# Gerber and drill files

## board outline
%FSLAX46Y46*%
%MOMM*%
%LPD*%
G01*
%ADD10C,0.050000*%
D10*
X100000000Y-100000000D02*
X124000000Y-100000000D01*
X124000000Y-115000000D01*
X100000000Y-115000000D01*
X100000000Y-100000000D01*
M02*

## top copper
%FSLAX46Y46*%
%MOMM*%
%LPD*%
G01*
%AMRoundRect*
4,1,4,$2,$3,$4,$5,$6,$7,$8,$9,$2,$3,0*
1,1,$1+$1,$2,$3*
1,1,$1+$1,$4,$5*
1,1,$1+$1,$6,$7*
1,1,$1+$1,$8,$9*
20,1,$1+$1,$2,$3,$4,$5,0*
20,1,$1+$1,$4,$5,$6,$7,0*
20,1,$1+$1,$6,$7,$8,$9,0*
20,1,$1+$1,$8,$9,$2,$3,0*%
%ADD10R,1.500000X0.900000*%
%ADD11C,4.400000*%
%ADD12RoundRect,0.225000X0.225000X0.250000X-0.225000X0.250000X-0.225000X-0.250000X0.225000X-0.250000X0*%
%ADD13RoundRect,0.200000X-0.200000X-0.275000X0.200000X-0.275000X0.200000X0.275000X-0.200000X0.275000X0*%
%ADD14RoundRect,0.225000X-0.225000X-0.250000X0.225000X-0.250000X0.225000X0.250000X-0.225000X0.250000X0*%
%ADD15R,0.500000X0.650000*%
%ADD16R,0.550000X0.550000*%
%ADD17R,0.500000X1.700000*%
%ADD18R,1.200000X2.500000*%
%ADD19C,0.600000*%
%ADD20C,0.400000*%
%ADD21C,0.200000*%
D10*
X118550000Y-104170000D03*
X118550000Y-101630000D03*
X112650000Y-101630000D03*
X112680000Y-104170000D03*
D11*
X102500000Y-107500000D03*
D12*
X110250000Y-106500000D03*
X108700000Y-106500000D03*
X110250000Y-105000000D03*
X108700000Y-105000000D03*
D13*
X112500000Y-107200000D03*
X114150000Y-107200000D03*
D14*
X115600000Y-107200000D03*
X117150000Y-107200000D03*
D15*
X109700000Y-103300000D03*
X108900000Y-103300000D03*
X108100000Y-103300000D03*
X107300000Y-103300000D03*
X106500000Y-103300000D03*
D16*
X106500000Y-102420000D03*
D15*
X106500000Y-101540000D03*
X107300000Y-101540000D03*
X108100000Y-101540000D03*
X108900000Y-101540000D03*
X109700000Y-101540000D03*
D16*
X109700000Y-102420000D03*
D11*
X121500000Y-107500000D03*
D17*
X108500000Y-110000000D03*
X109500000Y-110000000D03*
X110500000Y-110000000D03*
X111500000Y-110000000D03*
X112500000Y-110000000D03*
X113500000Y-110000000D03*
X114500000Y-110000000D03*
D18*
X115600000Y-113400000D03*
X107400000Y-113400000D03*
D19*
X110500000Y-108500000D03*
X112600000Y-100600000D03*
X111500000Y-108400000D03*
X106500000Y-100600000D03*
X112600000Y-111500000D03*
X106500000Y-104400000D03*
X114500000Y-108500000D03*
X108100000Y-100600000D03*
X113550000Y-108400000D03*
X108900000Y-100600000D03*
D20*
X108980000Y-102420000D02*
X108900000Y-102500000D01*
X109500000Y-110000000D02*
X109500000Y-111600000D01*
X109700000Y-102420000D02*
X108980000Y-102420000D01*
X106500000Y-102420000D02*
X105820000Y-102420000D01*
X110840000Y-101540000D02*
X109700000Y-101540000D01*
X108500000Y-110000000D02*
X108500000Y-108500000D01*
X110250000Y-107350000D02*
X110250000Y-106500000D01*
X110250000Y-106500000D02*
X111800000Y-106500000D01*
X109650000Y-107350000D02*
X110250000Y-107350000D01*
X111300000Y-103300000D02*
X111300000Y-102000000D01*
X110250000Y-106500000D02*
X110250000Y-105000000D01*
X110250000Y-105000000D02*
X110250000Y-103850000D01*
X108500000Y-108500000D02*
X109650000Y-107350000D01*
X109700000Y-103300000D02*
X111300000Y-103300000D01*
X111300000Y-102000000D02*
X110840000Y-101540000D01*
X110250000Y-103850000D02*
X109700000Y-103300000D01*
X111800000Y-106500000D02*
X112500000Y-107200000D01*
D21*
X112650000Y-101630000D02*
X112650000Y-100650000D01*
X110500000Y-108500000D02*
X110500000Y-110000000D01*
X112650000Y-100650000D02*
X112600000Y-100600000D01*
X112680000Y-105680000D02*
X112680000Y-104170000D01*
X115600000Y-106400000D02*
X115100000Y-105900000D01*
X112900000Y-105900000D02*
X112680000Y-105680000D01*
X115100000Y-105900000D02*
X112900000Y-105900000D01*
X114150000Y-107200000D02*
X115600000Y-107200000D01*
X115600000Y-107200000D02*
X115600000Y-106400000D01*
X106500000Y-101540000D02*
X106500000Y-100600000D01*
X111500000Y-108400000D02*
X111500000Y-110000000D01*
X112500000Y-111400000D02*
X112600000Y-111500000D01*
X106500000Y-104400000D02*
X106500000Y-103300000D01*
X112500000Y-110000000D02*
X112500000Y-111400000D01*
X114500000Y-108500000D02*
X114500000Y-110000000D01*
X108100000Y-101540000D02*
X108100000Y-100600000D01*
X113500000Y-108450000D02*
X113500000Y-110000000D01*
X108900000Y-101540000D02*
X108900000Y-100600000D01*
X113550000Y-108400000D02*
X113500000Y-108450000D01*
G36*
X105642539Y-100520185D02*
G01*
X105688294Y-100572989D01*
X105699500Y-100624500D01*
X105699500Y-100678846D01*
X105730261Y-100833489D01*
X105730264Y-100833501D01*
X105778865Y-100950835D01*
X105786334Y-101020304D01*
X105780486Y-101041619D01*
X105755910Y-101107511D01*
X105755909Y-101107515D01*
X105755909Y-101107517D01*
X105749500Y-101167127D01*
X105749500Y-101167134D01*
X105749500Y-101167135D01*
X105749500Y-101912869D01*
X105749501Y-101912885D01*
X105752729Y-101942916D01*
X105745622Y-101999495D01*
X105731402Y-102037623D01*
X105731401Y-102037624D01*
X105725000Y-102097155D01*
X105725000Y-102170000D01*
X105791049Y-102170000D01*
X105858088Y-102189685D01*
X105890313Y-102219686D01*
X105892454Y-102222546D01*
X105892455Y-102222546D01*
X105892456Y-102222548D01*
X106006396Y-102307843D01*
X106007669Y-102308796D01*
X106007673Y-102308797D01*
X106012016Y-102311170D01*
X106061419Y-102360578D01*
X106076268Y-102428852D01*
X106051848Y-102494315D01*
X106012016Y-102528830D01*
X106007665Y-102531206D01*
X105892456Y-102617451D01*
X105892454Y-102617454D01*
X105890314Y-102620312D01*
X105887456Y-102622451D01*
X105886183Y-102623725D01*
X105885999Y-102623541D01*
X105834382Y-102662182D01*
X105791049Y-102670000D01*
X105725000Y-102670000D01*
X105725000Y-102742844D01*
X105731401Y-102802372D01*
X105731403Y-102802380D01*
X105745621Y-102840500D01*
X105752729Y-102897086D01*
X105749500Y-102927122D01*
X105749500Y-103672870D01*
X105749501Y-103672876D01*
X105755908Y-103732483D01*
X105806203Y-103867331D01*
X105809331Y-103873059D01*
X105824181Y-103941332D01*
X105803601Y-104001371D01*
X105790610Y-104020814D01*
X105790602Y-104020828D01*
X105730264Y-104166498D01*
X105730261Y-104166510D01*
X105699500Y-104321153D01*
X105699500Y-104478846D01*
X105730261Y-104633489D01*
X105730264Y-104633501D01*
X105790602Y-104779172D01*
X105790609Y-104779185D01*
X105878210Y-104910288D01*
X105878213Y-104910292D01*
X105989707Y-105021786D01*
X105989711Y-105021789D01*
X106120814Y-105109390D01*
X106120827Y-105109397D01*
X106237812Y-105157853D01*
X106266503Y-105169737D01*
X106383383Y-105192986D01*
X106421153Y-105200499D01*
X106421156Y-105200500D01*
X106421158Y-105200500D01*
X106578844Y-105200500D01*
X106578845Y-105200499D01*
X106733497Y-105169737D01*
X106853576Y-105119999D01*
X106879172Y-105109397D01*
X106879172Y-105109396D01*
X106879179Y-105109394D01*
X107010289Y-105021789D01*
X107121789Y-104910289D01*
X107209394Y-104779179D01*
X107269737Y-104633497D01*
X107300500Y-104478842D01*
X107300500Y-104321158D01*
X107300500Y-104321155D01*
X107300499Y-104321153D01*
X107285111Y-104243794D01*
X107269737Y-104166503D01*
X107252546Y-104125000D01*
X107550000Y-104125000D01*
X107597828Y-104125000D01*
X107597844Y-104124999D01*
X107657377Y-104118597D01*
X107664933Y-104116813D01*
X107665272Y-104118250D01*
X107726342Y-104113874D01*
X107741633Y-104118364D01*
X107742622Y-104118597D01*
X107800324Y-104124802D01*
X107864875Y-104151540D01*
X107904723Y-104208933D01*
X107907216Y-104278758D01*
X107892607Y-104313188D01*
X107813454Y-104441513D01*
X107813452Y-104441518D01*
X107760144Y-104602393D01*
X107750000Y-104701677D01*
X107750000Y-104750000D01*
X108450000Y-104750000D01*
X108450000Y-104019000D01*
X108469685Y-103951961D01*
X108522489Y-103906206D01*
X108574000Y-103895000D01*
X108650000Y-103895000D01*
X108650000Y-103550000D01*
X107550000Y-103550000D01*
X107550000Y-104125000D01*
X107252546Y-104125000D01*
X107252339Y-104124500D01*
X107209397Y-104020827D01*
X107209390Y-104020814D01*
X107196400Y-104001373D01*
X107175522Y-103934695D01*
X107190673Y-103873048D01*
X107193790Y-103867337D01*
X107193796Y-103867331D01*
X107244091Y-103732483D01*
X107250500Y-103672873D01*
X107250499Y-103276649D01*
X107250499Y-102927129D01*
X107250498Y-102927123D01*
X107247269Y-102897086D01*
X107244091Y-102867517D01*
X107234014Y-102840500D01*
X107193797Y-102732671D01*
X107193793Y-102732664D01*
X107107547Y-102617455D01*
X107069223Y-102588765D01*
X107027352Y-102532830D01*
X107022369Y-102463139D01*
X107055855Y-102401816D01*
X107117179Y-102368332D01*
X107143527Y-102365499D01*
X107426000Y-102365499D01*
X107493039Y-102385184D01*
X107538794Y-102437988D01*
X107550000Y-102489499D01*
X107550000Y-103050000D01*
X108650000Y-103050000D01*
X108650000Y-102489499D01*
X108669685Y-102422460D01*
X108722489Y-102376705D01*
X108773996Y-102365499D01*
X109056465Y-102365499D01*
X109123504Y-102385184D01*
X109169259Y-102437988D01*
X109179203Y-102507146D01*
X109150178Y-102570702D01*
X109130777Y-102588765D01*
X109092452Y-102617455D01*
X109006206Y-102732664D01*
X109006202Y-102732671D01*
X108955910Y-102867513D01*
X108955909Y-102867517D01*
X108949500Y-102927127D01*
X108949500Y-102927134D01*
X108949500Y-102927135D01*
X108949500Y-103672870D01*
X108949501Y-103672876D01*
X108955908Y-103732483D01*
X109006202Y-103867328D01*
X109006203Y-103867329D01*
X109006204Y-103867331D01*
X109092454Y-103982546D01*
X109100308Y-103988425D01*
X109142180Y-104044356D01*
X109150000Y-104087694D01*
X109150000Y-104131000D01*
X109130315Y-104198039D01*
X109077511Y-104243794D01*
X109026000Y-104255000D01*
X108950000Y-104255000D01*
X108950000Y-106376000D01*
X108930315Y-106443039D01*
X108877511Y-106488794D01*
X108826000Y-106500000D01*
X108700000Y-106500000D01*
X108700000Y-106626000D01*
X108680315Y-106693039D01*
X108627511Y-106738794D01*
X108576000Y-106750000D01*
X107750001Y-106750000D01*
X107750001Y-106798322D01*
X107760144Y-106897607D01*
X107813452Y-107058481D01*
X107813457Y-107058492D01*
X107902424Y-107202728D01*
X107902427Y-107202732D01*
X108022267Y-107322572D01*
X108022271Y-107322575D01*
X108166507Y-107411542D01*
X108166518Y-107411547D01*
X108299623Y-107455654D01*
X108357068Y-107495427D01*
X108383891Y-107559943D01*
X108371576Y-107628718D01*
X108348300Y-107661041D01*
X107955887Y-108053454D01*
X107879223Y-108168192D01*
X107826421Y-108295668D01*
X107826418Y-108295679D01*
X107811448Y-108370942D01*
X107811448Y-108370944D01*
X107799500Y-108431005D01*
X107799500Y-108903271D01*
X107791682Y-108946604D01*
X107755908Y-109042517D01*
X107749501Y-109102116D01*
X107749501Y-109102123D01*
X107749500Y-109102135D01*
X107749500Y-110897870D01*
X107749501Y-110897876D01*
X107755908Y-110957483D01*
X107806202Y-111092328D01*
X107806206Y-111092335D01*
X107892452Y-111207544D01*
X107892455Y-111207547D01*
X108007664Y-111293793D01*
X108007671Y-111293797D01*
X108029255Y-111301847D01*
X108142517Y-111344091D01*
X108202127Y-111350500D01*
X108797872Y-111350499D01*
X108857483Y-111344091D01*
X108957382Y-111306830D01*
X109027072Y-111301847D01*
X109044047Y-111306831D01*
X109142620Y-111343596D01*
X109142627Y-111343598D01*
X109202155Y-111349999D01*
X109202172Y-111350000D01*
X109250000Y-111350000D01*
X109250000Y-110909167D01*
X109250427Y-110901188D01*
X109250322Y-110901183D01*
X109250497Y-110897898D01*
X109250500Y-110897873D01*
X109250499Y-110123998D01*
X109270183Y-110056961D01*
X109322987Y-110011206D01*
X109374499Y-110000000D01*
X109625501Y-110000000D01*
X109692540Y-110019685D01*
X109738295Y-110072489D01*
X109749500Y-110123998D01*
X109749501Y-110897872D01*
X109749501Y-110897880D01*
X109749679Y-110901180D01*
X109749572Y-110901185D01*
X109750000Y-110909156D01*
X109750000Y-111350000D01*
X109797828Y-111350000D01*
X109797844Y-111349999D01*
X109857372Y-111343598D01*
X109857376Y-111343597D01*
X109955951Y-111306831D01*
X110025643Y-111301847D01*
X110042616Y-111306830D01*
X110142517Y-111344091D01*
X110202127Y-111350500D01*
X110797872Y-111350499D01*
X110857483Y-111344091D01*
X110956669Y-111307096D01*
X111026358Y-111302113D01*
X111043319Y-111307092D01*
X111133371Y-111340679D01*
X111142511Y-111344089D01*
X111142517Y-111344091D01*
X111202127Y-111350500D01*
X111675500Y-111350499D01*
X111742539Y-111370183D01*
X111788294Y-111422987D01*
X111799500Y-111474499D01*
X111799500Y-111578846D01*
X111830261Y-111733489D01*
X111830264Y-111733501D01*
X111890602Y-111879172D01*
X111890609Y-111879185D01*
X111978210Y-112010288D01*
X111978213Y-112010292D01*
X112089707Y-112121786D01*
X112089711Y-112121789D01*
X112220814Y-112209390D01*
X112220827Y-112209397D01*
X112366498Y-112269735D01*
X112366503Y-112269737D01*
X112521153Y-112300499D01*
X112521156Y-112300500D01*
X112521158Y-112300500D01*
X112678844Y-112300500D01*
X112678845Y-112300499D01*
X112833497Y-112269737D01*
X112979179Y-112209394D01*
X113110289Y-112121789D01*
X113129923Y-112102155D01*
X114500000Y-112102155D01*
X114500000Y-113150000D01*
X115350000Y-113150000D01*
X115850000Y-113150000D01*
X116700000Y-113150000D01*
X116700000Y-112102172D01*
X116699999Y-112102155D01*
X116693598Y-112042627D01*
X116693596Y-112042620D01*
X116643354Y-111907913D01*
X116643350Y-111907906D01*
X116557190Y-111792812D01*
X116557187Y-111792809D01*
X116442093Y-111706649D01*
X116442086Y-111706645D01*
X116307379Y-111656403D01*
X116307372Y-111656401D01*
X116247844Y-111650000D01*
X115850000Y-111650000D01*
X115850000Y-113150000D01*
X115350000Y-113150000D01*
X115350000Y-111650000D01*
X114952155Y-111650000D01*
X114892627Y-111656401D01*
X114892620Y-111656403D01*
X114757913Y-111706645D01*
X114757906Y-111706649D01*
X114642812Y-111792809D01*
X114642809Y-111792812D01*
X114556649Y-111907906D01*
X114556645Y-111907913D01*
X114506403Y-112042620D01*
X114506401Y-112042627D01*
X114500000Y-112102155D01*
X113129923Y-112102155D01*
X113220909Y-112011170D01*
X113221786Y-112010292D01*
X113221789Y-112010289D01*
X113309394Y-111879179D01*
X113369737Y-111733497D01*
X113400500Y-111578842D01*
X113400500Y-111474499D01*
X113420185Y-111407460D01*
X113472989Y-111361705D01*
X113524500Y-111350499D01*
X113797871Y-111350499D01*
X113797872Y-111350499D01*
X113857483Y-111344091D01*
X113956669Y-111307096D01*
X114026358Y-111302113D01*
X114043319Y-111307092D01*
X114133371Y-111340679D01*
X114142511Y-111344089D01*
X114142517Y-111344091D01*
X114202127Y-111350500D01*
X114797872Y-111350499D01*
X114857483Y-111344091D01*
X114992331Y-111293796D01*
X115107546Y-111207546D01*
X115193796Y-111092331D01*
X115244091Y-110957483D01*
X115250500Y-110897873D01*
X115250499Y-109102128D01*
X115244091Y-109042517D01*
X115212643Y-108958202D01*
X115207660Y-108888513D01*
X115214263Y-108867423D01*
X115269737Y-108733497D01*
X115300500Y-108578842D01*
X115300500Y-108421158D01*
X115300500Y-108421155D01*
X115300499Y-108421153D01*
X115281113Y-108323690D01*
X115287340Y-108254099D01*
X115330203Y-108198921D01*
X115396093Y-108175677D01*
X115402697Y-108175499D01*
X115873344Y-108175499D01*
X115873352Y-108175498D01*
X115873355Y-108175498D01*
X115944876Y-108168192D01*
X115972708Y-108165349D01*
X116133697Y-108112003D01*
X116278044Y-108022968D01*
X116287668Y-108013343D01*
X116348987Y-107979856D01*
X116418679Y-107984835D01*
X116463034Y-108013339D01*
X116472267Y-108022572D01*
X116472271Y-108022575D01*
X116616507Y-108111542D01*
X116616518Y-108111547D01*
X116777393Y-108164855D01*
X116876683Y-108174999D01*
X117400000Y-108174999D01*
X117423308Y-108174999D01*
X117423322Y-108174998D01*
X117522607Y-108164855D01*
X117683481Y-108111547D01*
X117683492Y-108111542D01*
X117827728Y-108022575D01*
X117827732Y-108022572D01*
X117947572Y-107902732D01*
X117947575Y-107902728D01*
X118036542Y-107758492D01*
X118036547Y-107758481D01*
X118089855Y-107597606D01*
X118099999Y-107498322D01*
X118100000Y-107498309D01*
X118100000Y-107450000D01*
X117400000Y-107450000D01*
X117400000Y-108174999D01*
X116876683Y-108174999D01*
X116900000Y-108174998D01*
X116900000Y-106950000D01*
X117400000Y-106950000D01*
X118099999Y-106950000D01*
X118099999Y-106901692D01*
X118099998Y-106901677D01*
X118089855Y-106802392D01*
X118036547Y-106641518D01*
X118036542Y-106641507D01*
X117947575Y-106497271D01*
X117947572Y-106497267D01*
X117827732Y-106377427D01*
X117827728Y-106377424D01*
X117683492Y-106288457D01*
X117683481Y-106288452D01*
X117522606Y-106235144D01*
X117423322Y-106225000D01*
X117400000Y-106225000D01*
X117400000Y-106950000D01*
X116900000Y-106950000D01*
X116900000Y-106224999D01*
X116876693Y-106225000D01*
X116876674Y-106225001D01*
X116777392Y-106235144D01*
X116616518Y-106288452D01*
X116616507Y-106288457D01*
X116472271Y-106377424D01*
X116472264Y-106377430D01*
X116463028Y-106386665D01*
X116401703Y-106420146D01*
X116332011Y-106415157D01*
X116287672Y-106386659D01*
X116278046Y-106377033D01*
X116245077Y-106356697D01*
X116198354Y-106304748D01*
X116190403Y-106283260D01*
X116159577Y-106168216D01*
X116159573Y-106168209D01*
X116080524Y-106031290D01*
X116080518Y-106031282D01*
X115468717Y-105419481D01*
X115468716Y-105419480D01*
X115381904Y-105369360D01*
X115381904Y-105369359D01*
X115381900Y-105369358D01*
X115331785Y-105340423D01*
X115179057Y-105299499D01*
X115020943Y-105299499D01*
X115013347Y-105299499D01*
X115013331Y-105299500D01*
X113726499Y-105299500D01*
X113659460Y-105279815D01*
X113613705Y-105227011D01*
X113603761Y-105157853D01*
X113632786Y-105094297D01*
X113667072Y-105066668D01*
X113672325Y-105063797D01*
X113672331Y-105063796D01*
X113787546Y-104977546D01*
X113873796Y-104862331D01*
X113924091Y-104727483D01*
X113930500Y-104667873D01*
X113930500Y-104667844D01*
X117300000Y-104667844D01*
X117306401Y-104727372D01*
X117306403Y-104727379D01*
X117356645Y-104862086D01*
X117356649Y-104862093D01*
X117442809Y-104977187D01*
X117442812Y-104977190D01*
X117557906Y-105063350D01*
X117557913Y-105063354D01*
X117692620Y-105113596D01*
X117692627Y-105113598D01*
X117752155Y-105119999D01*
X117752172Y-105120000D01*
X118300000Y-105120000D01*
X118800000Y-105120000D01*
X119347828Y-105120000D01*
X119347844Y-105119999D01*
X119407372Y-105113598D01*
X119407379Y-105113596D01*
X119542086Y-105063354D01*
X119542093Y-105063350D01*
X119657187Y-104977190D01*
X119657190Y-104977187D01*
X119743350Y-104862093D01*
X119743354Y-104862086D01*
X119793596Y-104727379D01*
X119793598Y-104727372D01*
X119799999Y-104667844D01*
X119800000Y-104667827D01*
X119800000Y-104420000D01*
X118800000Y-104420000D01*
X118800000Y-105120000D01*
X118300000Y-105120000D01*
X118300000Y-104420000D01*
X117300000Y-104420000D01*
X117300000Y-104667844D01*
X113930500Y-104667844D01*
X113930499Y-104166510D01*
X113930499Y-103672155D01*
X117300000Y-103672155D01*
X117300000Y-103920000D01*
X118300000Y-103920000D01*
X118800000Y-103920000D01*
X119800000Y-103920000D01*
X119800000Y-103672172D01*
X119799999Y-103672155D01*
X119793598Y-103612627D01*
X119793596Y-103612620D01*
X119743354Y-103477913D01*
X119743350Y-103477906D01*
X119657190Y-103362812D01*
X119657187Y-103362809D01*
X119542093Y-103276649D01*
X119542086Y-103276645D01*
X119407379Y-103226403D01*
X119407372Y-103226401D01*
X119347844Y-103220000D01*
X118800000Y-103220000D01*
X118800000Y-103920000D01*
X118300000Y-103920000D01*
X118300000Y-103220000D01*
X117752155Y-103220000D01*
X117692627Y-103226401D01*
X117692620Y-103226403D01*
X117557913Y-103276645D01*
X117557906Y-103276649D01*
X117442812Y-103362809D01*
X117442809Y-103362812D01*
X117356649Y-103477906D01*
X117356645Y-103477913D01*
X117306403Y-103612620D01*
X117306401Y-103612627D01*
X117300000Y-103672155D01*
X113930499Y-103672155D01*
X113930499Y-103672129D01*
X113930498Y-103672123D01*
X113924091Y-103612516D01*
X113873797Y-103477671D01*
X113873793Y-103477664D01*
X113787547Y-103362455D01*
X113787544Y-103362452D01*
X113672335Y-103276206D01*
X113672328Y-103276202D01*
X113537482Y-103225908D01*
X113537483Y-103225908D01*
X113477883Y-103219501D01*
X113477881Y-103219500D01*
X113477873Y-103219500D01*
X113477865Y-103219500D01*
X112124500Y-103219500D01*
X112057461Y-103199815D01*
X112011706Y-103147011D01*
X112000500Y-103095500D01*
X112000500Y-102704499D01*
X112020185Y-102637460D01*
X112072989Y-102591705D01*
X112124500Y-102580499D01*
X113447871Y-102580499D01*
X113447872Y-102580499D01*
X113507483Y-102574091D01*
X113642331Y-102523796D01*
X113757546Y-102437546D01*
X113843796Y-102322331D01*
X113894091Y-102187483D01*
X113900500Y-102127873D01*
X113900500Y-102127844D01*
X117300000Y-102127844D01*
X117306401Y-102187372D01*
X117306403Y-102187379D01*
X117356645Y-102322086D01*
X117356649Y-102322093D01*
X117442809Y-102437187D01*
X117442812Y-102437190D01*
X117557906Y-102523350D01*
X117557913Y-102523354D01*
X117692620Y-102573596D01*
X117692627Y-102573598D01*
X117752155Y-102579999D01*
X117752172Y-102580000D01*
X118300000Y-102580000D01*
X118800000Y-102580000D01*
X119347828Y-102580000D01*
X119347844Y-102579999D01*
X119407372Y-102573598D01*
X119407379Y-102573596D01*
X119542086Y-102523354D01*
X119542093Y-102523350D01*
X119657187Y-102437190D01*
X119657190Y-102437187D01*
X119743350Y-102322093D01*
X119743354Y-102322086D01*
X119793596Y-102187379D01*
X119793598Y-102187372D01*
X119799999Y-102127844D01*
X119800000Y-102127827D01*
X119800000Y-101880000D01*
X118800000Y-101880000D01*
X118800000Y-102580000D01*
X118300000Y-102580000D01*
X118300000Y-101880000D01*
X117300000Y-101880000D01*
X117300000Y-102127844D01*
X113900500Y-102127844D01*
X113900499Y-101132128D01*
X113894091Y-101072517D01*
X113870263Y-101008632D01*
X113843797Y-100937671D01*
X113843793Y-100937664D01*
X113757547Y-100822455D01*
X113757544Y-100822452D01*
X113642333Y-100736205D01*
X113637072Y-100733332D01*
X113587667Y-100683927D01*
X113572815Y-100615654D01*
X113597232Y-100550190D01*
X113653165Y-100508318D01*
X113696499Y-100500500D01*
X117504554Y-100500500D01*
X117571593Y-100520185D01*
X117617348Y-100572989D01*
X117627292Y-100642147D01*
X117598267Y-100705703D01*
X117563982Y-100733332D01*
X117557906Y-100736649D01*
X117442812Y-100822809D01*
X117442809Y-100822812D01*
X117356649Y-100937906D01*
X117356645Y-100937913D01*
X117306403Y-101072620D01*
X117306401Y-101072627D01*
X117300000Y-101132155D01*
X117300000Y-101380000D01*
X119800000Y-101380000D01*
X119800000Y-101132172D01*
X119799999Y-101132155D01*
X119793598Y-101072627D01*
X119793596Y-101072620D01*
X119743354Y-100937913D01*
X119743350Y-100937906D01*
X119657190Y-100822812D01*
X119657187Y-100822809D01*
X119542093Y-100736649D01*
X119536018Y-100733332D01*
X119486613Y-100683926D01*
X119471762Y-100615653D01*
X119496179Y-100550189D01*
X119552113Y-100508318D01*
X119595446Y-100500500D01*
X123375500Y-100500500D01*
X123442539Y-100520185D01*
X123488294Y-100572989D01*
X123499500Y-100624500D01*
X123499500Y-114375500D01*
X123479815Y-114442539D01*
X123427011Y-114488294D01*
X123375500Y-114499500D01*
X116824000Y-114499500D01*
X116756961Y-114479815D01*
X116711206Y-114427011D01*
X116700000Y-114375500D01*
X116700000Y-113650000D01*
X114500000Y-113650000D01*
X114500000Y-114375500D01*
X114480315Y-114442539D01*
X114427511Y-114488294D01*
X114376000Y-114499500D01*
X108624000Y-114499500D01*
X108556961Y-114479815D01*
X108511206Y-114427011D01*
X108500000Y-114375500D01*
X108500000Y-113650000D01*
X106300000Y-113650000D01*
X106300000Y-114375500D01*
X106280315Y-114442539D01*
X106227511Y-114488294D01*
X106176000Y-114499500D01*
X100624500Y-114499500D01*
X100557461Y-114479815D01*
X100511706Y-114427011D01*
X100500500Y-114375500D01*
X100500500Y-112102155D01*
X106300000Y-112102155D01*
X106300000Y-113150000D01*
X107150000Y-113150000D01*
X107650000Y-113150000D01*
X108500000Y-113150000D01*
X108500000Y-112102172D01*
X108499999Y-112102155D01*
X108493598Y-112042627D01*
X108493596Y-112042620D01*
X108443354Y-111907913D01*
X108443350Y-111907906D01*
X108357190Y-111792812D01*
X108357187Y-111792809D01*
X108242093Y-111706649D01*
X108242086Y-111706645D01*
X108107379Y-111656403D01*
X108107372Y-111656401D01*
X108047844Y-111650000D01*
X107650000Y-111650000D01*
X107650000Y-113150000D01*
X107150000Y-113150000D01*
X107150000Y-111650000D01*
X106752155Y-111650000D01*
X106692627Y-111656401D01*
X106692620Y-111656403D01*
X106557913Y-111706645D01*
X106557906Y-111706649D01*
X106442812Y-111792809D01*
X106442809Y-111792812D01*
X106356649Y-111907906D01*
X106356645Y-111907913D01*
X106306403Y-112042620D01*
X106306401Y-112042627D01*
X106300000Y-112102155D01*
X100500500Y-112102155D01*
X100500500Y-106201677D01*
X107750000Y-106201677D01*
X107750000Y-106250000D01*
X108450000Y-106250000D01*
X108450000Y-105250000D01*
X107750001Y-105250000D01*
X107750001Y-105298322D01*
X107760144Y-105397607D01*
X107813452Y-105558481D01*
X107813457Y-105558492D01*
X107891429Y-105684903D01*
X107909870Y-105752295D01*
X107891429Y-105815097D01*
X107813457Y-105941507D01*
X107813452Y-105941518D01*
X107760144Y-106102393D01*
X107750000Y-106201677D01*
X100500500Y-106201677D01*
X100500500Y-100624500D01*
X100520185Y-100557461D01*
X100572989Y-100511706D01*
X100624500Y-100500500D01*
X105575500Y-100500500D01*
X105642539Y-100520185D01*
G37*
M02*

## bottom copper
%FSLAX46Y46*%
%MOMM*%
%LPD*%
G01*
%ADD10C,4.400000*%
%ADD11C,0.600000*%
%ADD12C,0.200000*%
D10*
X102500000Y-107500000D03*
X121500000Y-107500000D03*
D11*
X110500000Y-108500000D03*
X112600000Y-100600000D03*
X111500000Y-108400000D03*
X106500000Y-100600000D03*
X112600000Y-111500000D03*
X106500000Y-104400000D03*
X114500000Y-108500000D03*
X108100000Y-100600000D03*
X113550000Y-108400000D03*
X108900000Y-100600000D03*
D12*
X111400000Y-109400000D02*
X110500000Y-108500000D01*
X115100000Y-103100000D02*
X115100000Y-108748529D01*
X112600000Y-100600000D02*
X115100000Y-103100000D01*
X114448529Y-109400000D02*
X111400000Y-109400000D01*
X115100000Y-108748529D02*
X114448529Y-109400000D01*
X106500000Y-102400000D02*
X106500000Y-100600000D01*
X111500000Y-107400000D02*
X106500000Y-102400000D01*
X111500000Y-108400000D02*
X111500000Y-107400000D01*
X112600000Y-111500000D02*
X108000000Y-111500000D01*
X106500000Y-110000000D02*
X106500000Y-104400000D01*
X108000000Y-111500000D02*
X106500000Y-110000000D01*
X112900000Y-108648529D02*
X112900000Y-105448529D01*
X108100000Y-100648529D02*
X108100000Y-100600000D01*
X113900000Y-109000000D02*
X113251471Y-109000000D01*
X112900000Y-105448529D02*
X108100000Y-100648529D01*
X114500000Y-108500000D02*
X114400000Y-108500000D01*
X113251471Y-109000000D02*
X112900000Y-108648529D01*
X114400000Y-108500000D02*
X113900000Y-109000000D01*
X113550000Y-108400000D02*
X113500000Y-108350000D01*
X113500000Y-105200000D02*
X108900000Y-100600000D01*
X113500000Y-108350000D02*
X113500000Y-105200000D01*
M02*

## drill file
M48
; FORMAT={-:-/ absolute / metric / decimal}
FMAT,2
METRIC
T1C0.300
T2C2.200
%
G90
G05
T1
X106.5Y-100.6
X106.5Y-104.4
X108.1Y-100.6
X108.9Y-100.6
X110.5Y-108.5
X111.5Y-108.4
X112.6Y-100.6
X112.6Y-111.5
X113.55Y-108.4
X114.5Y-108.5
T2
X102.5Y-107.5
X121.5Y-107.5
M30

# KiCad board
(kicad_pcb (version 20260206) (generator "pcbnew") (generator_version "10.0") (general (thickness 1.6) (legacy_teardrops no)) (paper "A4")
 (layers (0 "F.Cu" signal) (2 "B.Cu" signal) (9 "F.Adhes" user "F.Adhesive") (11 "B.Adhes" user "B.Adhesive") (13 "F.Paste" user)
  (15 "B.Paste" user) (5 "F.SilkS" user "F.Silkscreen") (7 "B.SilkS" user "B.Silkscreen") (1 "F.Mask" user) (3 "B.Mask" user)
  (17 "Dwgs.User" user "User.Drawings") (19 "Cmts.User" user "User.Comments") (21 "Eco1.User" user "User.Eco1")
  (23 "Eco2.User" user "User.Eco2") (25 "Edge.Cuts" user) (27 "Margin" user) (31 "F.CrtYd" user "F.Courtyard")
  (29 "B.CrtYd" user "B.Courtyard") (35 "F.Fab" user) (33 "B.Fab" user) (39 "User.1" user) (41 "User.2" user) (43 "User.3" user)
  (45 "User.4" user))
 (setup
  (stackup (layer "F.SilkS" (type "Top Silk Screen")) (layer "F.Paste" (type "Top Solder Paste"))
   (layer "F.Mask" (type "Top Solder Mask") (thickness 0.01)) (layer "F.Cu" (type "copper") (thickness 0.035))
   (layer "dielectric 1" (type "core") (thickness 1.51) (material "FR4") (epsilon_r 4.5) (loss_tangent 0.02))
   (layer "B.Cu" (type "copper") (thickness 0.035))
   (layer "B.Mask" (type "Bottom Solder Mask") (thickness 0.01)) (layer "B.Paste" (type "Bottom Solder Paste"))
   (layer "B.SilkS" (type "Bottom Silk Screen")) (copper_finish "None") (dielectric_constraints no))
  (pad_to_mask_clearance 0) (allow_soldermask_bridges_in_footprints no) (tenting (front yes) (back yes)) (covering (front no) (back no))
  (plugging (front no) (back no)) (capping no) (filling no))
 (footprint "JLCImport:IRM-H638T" (layer "F.Cu") (at 115.6 102.9 180)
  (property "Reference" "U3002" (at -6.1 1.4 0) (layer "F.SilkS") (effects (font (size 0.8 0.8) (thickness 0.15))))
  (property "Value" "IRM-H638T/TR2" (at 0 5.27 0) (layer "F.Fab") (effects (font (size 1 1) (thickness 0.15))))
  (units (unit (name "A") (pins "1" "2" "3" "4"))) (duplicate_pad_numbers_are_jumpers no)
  (pad "1" smd rect (at -2.95 -1.27 270) (size 0.9 1.5) (layers "F.Cu" "F.Mask" "F.Paste") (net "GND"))
  (pad "2" smd rect (at -2.95 1.27 270) (size 0.9 1.5) (layers "F.Cu" "F.Mask" "F.Paste") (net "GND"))
  (pad "3" smd rect (at 2.95 1.27 270) (size 0.9 1.5) (layers "F.Cu" "F.Mask" "F.Paste") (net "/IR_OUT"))
  (pad "4" smd rect (at 2.92 -1.27 270) (size 0.9 1.5) (layers "F.Cu" "F.Mask" "F.Paste") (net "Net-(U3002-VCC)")))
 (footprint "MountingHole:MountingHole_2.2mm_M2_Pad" (layer "F.Cu") (at 102.5 107.5)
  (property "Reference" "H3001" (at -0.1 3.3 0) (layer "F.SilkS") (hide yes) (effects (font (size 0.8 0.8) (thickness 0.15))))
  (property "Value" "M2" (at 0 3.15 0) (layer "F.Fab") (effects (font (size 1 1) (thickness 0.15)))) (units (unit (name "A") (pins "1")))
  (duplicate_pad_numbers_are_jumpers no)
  (pad "1" thru_hole circle (at 0 0) (size 4.4 4.4) (drill 2.2) (layers "*.Cu" "*.Mask") (remove_unused_layers no) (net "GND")
   (zone_connect 2)))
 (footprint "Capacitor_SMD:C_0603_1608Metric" (layer "F.Cu") (at 109.475 106.5 180)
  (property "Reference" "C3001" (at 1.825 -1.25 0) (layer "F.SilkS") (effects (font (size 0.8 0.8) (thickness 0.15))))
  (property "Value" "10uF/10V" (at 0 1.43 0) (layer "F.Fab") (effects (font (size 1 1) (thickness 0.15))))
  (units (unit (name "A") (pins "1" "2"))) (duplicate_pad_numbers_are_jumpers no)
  (pad "1" smd roundrect (at -0.775 0 180) (size 0.9 0.95) (layers "F.Cu" "F.Mask" "F.Paste") (roundrect_rratio 0.25) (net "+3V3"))
  (pad "2" smd roundrect (at 0.775 0 180) (size 0.9 0.95) (layers "F.Cu" "F.Mask" "F.Paste") (roundrect_rratio 0.25) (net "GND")))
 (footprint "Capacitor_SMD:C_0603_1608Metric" (layer "F.Cu") (at 109.475 105 180)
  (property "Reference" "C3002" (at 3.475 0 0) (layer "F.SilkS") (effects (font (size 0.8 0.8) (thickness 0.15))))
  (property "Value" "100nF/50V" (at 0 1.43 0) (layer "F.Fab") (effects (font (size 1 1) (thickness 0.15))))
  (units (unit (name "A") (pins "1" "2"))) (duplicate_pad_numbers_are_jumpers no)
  (pad "1" smd roundrect (at -0.775 0 180) (size 0.9 0.95) (layers "F.Cu" "F.Mask" "F.Paste") (roundrect_rratio 0.25) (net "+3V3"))
  (pad "2" smd roundrect (at 0.775 0 180) (size 0.9 0.95) (layers "F.Cu" "F.Mask" "F.Paste") (roundrect_rratio 0.25) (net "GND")))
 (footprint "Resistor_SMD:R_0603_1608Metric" (layer "F.Cu") (at 113.325 107.2)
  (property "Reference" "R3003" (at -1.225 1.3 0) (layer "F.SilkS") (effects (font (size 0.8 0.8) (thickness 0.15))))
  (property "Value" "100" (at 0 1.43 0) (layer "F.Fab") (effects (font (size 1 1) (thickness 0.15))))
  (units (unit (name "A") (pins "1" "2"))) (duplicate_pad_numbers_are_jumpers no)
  (pad "1" smd roundrect (at -0.825 0) (size 0.8 0.95) (layers "F.Cu" "F.Mask" "F.Paste") (roundrect_rratio 0.25) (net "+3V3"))
  (pad "2" smd roundrect (at 0.825 0) (size 0.8 0.95) (layers "F.Cu" "F.Mask" "F.Paste") (roundrect_rratio 0.25) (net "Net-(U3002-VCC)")))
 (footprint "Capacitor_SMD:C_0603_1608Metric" (layer "F.Cu") (at 116.375 107.2)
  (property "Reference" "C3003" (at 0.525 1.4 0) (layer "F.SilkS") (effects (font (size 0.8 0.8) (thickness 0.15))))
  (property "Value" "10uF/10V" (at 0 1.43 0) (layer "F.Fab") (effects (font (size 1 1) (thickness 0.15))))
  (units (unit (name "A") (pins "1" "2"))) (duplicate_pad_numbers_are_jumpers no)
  (pad "1" smd roundrect (at -0.775 0) (size 0.9 0.95) (layers "F.Cu" "F.Mask" "F.Paste") (roundrect_rratio 0.25) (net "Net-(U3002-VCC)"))
  (pad "2" smd roundrect (at 0.775 0) (size 0.9 0.95) (layers "F.Cu" "F.Mask" "F.Paste") (roundrect_rratio 0.25) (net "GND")))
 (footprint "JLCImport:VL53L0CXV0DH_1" (layer "F.Cu") (at 108.1 102.42)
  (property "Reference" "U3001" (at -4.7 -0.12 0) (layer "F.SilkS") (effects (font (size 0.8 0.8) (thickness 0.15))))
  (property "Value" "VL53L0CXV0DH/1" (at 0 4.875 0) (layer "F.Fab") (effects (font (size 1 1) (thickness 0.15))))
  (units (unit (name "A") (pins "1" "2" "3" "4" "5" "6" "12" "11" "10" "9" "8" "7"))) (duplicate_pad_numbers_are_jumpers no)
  (pad "1" smd rect (at 1.6 0.88) (size 0.5 0.65) (layers "F.Cu" "F.Mask" "F.Paste") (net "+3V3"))
  (pad "2" smd rect (at 0.8 0.88) (size 0.5 0.65) (layers "F.Cu" "F.Mask" "F.Paste") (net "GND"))
  (pad "3" smd rect (at 0 0.88) (size 0.5 0.65) (layers "F.Cu" "F.Mask" "F.Paste") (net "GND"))
  (pad "4" smd rect (at -0.8 0.88) (size 0.5 0.65) (layers "F.Cu" "F.Mask" "F.Paste") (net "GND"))
  (pad "5" smd rect (at -1.6 0.88) (size 0.5 0.65) (layers "F.Cu" "F.Mask" "F.Paste") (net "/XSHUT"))
  (pad "6" smd rect (at -1.6 0) (size 0.55 0.55) (layers "F.Cu" "F.Mask" "F.Paste") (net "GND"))
  (pad "7" smd rect (at -1.6 -0.88) (size 0.5 0.65) (layers "F.Cu" "F.Mask" "F.Paste") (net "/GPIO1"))
  (pad "8" smd rect (at -0.8 -0.88) (size 0.5 0.65) (layers "F.Cu" "F.Mask" "F.Paste") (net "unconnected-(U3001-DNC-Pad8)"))
  (pad "9" smd rect (at 0 -0.88) (size 0.5 0.65) (layers "F.Cu" "F.Mask" "F.Paste") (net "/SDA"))
  (pad "10" smd rect (at 0.8 -0.88) (size 0.5 0.65) (layers "F.Cu" "F.Mask" "F.Paste") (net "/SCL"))
  (pad "11" smd rect (at 1.6 -0.88) (size 0.5 0.65) (layers "F.Cu" "F.Mask" "F.Paste") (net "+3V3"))
  (pad "12" smd rect (at 1.6 0) (size 0.55 0.55) (layers "F.Cu" "F.Mask" "F.Paste") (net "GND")))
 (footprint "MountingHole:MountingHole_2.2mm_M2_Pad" (layer "F.Cu") (at 121.5 107.5)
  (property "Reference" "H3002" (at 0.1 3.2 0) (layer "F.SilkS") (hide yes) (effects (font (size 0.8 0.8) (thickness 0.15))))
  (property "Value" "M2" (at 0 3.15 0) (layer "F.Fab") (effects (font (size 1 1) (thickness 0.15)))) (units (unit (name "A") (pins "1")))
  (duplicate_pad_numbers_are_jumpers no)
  (pad "1" thru_hole circle (at 0 0) (size 4.4 4.4) (drill 2.2) (layers "*.Cu" "*.Mask") (remove_unused_layers no) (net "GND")
   (zone_connect 2)))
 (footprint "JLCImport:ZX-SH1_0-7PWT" (layer "F.Cu") (at 111.5 111.7)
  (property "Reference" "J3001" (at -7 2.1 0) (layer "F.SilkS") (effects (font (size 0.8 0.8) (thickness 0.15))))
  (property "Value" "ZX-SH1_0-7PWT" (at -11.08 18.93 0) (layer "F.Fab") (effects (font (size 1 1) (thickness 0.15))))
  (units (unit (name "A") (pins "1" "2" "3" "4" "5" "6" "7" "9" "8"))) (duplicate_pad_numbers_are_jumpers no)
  (pad "1" smd rect (at -3 -1.7) (size 0.5 1.7) (layers "F.Cu" "F.Mask" "F.Paste") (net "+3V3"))
  (pad "2" smd rect (at -2 -1.7) (size 0.5 1.7) (layers "F.Cu" "F.Mask" "F.Paste") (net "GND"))
  (pad "3" smd rect (at -1 -1.7) (size 0.5 1.7) (layers "F.Cu" "F.Mask" "F.Paste") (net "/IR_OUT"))
  (pad "4" smd rect (at 0 -1.7) (size 0.5 1.7) (layers "F.Cu" "F.Mask" "F.Paste") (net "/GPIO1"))
  (pad "5" smd rect (at 1 -1.7) (size 0.5 1.7) (layers "F.Cu" "F.Mask" "F.Paste") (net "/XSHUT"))
  (pad "6" smd rect (at 2 -1.7) (size 0.5 1.7) (layers "F.Cu" "F.Mask" "F.Paste") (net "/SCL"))
  (pad "7" smd rect (at 3 -1.7) (size 0.5 1.7) (layers "F.Cu" "F.Mask" "F.Paste") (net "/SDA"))
  (pad "8" smd rect (at 4.1 1.7) (size 1.2 2.5) (layers "F.Cu" "F.Mask" "F.Paste") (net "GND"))
  (pad "9" smd rect (at -4.1 1.7) (size 1.2 2.5) (layers "F.Cu" "F.Mask" "F.Paste") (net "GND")))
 (gr_rect (start 100 100) (end 124 115) (stroke (width 0.05) (type solid)) (fill no) (layer "Edge.Cuts"))
 (segment (start 108.98 102.42) (end 108.9 102.5) (width 0.4) (layer "F.Cu") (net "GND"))
 (segment (start 109.5 110) (end 109.5 111.6) (width 0.4) (layer "F.Cu") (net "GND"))
 (segment (start 109.7 102.42) (end 108.98 102.42) (width 0.4) (layer "F.Cu") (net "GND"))
 (segment (start 106.5 102.42) (end 105.82 102.42) (width 0.4) (layer "F.Cu") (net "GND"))
 (segment (start 110.84 101.54) (end 109.7 101.54) (width 0.4) (layer "F.Cu") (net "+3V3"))
 (segment (start 108.5 110) (end 108.5 108.5) (width 0.4) (layer "F.Cu") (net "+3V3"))
 (segment (start 110.25 107.35) (end 110.25 106.5) (width 0.4) (layer "F.Cu") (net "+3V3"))
 (segment (start 110.25 106.5) (end 111.8 106.5) (width 0.4) (layer "F.Cu") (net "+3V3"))
 (segment (start 109.65 107.35) (end 110.25 107.35) (width 0.4) (layer "F.Cu") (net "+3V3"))
 (segment (start 111.3 103.3) (end 111.3 102) (width 0.4) (layer "F.Cu") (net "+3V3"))
 (segment (start 110.25 106.5) (end 110.25 105) (width 0.4) (layer "F.Cu") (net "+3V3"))
 (segment (start 110.25 105) (end 110.25 103.85) (width 0.4) (layer "F.Cu") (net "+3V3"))
 (segment (start 108.5 108.5) (end 109.65 107.35) (width 0.4) (layer "F.Cu") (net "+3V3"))
 (segment (start 109.7 103.3) (end 111.3 103.3) (width 0.4) (layer "F.Cu") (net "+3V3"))
 (segment (start 111.3 102) (end 110.84 101.54) (width 0.4) (layer "F.Cu") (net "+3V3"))
 (segment (start 110.25 103.85) (end 109.7 103.3) (width 0.4) (layer "F.Cu") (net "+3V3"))
 (segment (start 111.8 106.5) (end 112.5 107.2) (width 0.4) (layer "F.Cu") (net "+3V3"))
 (segment (start 112.65 101.63) (end 112.65 100.65) (width 0.2) (layer "F.Cu") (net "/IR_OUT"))
 (segment (start 110.5 108.5) (end 110.5 110) (width 0.2) (layer "F.Cu") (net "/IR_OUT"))
 (segment (start 112.65 100.65) (end 112.6 100.6) (width 0.2) (layer "F.Cu") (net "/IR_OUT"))
 (via (at 110.5 108.5) (size 0.6) (drill 0.3) (layers "F.Cu" "B.Cu") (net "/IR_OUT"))
 (via (at 112.6 100.6) (size 0.6) (drill 0.3) (layers "F.Cu" "B.Cu") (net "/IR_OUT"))
 (segment (start 111.4 109.4) (end 110.5 108.5) (width 0.2) (layer "B.Cu") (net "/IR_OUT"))
 (segment (start 115.1 103.1) (end 115.1 108.748529) (width 0.2) (layer "B.Cu") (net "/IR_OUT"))
 (segment (start 112.6 100.6) (end 115.1 103.1) (width 0.2) (layer "B.Cu") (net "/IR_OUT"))
 (segment (start 114.448529 109.4) (end 111.4 109.4) (width 0.2) (layer "B.Cu") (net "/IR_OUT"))
 (segment (start 115.1 108.748529) (end 114.448529 109.4) (width 0.2) (layer "B.Cu") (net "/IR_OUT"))
 (segment (start 112.68 105.68) (end 112.68 104.17) (width 0.2) (layer "F.Cu") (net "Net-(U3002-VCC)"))
 (segment (start 115.6 106.4) (end 115.1 105.9) (width 0.2) (layer "F.Cu") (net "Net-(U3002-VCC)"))
 (segment (start 112.9 105.9) (end 112.68 105.68) (width 0.2) (layer "F.Cu") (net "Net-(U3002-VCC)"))
 (segment (start 115.1 105.9) (end 112.9 105.9) (width 0.2) (layer "F.Cu") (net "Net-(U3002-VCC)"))
 (segment (start 114.15 107.2) (end 115.6 107.2) (width 0.2) (layer "F.Cu") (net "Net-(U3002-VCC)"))
 (segment (start 115.6 107.2) (end 115.6 106.4) (width 0.2) (layer "F.Cu") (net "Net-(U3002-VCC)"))
 (segment (start 106.5 101.54) (end 106.5 100.6) (width 0.2) (layer "F.Cu") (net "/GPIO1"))
 (segment (start 111.5 108.4) (end 111.5 110) (width 0.2) (layer "F.Cu") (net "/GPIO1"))
 (via (at 111.5 108.4) (size 0.6) (drill 0.3) (layers "F.Cu" "B.Cu") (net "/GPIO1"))
 (via (at 106.5 100.6) (size 0.6) (drill 0.3) (layers "F.Cu" "B.Cu") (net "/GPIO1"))
 (segment (start 106.5 102.4) (end 106.5 100.6) (width 0.2) (layer "B.Cu") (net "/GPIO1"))
 (segment (start 111.5 107.4) (end 106.5 102.4) (width 0.2) (layer "B.Cu") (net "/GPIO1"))
 (segment (start 111.5 108.4) (end 111.5 107.4) (width 0.2) (layer "B.Cu") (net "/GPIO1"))
 (segment (start 112.5 111.4) (end 112.6 111.5) (width 0.2) (layer "F.Cu") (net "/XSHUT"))
 (segment (start 106.5 104.4) (end 106.5 103.3) (width 0.2) (layer "F.Cu") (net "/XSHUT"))
 (segment (start 112.5 110) (end 112.5 111.4) (width 0.2) (layer "F.Cu") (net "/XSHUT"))
 (via (at 112.6 111.5) (size 0.6) (drill 0.3) (layers "F.Cu" "B.Cu") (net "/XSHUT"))
 (via (at 106.5 104.4) (size 0.6) (drill 0.3) (layers "F.Cu" "B.Cu") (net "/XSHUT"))
 (segment (start 112.6 111.5) (end 108 111.5) (width 0.2) (layer "B.Cu") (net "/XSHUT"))
 (segment (start 106.5 110) (end 106.5 104.4) (width 0.2) (layer "B.Cu") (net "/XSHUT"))
 (segment (start 108 111.5) (end 106.5 110) (width 0.2) (layer "B.Cu") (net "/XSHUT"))
 (segment (start 114.5 108.5) (end 114.5 110) (width 0.2) (layer "F.Cu") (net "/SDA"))
 (segment (start 108.1 101.54) (end 108.1 100.6) (width 0.2) (layer "F.Cu") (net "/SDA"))
 (via (at 114.5 108.5) (size 0.6) (drill 0.3) (layers "F.Cu" "B.Cu") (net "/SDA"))
 (via (at 108.1 100.6) (size 0.6) (drill 0.3) (layers "F.Cu" "B.Cu") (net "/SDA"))
 (segment (start 112.9 108.648529) (end 112.9 105.448529) (width 0.2) (layer "B.Cu") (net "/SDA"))
 (segment (start 108.1 100.648529) (end 108.1 100.6) (width 0.2) (layer "B.Cu") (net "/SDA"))
 (segment (start 113.9 109) (end 113.251471 109) (width 0.2) (layer "B.Cu") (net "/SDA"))
 (segment (start 112.9 105.448529) (end 108.1 100.648529) (width 0.2) (layer "B.Cu") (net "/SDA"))
 (segment (start 114.5 108.5) (end 114.4 108.5) (width 0.2) (layer "B.Cu") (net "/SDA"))
 (segment (start 113.251471 109) (end 112.9 108.648529) (width 0.2) (layer "B.Cu") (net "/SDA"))
 (segment (start 114.4 108.5) (end 113.9 109) (width 0.2) (layer "B.Cu") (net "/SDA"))
 (segment (start 113.5 108.45) (end 113.5 110) (width 0.2) (layer "F.Cu") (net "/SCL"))
 (segment (start 108.9 101.54) (end 108.9 100.6) (width 0.2) (layer "F.Cu") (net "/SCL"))
 (segment (start 113.55 108.4) (end 113.5 108.45) (width 0.2) (layer "F.Cu") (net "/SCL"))
 (via (at 113.55 108.4) (size 0.6) (drill 0.3) (layers "F.Cu" "B.Cu") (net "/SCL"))
 (via (at 108.9 100.6) (size 0.6) (drill 0.3) (layers "F.Cu" "B.Cu") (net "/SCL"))
 (segment (start 113.55 108.4) (end 113.5 108.35) (width 0.2) (layer "B.Cu") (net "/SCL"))
 (segment (start 113.5 105.2) (end 108.9 100.6) (width 0.2) (layer "B.Cu") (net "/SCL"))
 (segment (start 113.5 108.35) (end 113.5 105.2) (width 0.2) (layer "B.Cu") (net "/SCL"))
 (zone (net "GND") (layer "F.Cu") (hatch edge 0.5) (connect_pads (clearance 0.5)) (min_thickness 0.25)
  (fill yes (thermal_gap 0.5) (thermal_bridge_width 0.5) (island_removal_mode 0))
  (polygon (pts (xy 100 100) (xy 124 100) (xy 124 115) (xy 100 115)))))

